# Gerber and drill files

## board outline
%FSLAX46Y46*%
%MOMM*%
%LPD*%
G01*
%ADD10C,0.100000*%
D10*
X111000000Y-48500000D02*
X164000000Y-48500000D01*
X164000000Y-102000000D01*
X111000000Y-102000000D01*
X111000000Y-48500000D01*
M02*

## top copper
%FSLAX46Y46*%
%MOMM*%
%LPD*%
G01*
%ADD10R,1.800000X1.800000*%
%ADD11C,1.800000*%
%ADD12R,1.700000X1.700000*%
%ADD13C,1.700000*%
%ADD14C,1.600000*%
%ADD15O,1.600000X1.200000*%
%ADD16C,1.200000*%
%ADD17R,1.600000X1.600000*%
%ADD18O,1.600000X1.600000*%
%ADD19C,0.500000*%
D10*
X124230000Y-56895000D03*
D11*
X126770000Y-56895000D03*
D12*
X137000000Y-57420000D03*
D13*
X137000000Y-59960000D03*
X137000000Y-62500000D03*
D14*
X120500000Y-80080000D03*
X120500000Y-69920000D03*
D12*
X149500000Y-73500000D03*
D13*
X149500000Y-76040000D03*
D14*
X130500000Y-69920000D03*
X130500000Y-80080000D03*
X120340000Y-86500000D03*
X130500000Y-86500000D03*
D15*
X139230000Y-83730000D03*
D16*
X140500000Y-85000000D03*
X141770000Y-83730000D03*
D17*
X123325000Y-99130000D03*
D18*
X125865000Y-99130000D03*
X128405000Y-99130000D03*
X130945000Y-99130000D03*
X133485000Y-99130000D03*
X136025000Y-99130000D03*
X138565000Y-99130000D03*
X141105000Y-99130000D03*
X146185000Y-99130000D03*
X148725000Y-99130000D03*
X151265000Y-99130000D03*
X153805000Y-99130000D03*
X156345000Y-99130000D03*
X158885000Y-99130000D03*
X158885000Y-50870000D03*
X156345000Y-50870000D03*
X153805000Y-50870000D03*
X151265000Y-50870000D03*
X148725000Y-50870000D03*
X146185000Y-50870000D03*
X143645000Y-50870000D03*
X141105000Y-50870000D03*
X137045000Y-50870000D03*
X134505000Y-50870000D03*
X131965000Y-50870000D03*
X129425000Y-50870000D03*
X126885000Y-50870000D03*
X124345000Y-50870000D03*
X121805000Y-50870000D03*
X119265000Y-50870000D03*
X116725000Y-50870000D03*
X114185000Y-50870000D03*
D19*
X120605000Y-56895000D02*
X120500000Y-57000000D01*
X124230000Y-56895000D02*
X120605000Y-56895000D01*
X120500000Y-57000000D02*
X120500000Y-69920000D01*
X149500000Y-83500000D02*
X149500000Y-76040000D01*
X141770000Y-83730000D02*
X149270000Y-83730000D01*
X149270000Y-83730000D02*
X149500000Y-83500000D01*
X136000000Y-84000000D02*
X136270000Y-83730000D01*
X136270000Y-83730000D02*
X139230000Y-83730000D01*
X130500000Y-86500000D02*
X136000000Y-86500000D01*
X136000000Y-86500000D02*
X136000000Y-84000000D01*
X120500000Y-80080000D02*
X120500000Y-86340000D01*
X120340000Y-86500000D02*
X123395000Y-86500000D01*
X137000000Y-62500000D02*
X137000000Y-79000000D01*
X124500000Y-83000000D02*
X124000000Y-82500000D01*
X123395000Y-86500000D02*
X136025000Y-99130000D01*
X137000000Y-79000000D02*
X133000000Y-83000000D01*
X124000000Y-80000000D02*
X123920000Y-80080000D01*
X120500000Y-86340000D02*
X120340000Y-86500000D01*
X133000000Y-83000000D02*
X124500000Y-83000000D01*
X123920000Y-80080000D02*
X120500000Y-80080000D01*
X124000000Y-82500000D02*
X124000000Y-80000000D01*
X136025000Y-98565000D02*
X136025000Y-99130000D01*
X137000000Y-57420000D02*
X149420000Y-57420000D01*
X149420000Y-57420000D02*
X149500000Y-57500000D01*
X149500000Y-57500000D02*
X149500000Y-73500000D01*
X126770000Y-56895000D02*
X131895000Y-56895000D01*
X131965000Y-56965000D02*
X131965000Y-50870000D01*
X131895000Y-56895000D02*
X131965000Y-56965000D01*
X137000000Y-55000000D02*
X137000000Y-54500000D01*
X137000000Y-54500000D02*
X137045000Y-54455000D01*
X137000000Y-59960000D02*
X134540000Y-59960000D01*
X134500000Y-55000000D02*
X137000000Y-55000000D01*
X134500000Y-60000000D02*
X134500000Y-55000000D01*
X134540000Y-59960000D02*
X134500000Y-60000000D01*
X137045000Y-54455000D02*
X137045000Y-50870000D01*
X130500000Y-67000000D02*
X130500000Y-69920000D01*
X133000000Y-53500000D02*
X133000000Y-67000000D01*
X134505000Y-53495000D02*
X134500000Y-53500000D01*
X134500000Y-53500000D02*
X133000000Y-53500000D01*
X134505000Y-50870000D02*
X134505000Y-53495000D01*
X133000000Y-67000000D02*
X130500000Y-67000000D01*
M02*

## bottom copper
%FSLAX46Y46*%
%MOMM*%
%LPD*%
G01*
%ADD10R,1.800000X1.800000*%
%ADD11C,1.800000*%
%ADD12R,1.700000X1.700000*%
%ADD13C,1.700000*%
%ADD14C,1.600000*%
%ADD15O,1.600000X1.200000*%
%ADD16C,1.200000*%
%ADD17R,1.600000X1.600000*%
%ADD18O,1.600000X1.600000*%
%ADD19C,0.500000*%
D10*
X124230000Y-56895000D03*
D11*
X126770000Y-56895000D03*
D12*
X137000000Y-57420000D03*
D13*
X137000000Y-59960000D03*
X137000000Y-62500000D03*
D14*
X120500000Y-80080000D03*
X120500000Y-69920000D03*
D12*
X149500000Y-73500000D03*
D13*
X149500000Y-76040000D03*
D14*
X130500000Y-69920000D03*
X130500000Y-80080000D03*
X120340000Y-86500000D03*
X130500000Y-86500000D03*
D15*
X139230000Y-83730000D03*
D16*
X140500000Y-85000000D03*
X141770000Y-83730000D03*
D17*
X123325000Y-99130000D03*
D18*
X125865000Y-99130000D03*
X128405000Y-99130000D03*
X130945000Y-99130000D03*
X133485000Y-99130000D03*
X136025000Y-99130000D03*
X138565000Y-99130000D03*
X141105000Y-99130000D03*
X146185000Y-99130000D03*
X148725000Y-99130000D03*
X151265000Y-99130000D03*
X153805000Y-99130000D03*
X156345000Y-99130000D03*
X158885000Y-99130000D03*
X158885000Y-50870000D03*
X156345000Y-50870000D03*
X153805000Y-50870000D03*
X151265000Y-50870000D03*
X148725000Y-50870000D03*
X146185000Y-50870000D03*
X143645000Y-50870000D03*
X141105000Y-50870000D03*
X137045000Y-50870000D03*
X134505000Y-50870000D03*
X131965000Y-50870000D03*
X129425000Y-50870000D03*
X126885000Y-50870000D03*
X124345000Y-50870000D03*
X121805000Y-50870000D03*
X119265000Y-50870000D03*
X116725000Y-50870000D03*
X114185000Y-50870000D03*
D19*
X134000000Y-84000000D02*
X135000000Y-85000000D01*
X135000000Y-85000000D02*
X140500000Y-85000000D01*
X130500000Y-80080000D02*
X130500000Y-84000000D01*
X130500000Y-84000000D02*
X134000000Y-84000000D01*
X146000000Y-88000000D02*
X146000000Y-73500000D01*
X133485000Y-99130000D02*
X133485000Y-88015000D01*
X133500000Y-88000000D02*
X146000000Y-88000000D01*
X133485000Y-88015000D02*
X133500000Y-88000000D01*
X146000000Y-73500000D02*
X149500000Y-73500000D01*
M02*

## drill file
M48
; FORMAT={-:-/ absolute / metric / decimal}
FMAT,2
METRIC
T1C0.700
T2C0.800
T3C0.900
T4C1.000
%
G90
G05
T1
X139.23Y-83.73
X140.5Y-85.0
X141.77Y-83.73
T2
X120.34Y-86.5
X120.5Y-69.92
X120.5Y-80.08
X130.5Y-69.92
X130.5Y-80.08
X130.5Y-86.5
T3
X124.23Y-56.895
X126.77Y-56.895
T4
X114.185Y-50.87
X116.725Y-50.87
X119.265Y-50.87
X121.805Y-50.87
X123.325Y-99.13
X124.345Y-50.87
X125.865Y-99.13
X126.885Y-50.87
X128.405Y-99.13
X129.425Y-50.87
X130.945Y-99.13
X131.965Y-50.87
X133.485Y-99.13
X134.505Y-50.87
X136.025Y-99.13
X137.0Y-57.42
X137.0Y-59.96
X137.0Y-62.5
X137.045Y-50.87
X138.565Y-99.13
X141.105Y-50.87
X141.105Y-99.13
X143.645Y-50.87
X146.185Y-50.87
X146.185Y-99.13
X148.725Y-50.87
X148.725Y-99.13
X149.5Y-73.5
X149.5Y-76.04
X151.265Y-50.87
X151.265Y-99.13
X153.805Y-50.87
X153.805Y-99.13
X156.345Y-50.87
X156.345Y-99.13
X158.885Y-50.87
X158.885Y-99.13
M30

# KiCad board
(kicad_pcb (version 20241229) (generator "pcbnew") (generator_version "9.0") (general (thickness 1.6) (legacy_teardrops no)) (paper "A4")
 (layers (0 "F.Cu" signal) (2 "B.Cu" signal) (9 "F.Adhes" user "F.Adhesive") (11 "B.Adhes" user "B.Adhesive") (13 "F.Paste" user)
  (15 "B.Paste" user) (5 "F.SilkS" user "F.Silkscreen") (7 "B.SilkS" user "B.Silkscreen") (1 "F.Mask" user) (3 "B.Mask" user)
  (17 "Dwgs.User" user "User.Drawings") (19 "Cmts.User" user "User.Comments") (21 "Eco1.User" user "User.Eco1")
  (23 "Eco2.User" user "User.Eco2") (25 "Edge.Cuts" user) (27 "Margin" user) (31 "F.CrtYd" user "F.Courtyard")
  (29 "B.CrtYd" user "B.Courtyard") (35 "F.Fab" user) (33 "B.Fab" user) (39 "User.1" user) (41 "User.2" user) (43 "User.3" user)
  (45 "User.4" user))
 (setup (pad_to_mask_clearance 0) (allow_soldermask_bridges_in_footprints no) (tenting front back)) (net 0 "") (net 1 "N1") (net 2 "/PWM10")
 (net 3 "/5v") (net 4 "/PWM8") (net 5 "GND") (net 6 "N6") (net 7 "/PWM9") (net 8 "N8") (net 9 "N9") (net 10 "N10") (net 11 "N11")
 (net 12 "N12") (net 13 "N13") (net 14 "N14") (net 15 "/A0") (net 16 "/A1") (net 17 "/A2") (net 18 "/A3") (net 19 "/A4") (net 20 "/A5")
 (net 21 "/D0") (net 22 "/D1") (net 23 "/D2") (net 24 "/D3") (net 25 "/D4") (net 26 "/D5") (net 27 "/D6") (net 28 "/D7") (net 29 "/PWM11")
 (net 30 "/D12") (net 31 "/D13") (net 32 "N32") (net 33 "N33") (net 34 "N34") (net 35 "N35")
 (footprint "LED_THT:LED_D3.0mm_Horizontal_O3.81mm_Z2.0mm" (layer "F.Cu") (at 124.23 56.895)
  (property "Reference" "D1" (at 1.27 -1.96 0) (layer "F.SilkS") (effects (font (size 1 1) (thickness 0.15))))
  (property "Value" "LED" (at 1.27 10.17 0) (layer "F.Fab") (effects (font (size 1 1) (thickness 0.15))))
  (pad "1" thru_hole rect (at 0 0) (size 1.8 1.8) (drill 0.9) (layers "*.Cu" "*.Mask") (remove_unused_layers no) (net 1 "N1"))
  (pad "2" thru_hole circle (at 2.54 0) (size 1.8 1.8) (drill 0.9) (layers "*.Cu" "*.Mask") (remove_unused_layers no) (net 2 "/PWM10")))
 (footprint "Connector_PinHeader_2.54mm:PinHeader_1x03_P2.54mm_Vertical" (layer "F.Cu") (at 137 57.42)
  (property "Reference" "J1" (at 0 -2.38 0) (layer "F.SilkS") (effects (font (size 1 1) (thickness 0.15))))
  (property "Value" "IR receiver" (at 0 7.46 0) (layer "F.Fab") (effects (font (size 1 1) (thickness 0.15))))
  (pad "1" thru_hole rect (at 0 0) (size 1.7 1.7) (drill 1) (layers "*.Cu" "*.Mask") (remove_unused_layers no) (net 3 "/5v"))
  (pad "2" thru_hole circle (at 0 2.54) (size 1.7 1.7) (drill 1) (layers "*.Cu" "*.Mask") (remove_unused_layers no) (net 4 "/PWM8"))
  (pad "3" thru_hole circle (at 0 5.08) (size 1.7 1.7) (drill 1) (layers "*.Cu" "*.Mask") (remove_unused_layers no) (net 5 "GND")))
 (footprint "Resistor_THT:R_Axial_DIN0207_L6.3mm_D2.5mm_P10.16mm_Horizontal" (layer "F.Cu") (at 120.5 80.08 90)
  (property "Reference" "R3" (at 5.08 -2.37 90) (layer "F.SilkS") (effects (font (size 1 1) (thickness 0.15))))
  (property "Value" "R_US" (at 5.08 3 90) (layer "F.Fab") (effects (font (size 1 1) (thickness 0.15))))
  (pad "1" thru_hole circle (at 0 0 90) (size 1.6 1.6) (drill 0.8) (layers "*.Cu" "*.Mask") (remove_unused_layers no) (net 5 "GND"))
  (pad "2" thru_hole circle (at 10.16 0 90) (size 1.6 1.6) (drill 0.8) (layers "*.Cu" "*.Mask") (remove_unused_layers no) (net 1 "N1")))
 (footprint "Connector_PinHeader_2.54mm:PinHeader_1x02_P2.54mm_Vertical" (layer "F.Cu") (at 149.5 73.5)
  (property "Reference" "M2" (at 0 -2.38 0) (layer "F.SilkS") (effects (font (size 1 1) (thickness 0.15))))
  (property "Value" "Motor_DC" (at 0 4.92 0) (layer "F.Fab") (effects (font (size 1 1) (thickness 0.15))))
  (pad "1" thru_hole rect (at 0 0) (size 1.7 1.7) (drill 1) (layers "*.Cu" "*.Mask") (remove_unused_layers no) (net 3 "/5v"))
  (pad "2" thru_hole circle (at 0 2.54) (size 1.7 1.7) (drill 1) (layers "*.Cu" "*.Mask") (remove_unused_layers no) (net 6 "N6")))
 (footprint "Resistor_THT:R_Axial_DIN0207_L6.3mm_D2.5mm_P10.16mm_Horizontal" (layer "F.Cu") (at 130.5 69.92 -90)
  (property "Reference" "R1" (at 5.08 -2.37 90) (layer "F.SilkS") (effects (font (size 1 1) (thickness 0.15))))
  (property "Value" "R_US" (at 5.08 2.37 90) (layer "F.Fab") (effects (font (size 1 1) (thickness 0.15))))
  (pad "1" thru_hole circle (at 0 0 270) (size 1.6 1.6) (drill 0.8) (layers "*.Cu" "*.Mask") (remove_unused_layers no) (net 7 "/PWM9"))
  (pad "2" thru_hole circle (at 10.16 0 270) (size 1.6 1.6) (drill 0.8) (layers "*.Cu" "*.Mask") (remove_unused_layers no) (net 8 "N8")))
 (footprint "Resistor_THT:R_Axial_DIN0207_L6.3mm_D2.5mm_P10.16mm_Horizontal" (layer "F.Cu") (at 120.34 86.5)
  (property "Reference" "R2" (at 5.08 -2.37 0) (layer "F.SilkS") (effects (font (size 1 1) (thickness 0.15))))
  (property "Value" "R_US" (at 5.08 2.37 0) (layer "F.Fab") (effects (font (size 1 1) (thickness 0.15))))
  (pad "1" thru_hole circle (at 0 0) (size 1.6 1.6) (drill 0.8) (layers "*.Cu" "*.Mask") (remove_unused_layers no) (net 5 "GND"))
  (pad "2" thru_hole circle (at 10.16 0) (size 1.6 1.6) (drill 0.8) (layers "*.Cu" "*.Mask") (remove_unused_layers no) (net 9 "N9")))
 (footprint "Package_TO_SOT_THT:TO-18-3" (layer "F.Cu") (at 139.23 83.73)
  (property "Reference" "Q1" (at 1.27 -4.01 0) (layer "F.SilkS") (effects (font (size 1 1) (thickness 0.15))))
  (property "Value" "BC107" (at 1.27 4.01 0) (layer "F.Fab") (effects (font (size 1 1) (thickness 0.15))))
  (pad "1" thru_hole oval (at 0 0) (size 1.6 1.2) (drill 0.7) (layers "*.Cu" "*.Mask") (remove_unused_layers no) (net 9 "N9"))
  (pad "2" thru_hole circle (at 1.27 1.27) (size 1.2 1.2) (drill 0.7) (layers "*.Cu" "*.Mask") (remove_unused_layers no) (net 8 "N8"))
  (pad "3" thru_hole circle (at 2.54 0) (size 1.2 1.2) (drill 0.7) (layers "*.Cu" "*.Mask") (remove_unused_layers no) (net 6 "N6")))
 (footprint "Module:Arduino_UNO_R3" (layer "B.Cu") (at 123.325 99.13)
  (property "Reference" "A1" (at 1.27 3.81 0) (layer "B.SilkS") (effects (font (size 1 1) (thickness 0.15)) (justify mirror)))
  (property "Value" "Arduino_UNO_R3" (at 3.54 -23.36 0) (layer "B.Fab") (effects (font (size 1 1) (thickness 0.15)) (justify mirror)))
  (pad "1" thru_hole rect (at 0 0 270) (size 1.6 1.6) (drill 1) (layers "*.Cu" "*.Mask") (remove_unused_layers no) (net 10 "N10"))
  (pad "2" thru_hole oval (at 2.54 0 270) (size 1.6 1.6) (drill 1) (layers "*.Cu" "*.Mask") (remove_unused_layers no) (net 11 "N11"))
  (pad "3" thru_hole oval (at 5.08 0 270) (size 1.6 1.6) (drill 1) (layers "*.Cu" "*.Mask") (remove_unused_layers no) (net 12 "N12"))
  (pad "4" thru_hole oval (at 7.62 0 270) (size 1.6 1.6) (drill 1) (layers "*.Cu" "*.Mask") (remove_unused_layers no) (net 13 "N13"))
  (pad "5" thru_hole oval (at 10.16 0 270) (size 1.6 1.6) (drill 1) (layers "*.Cu" "*.Mask") (remove_unused_layers no) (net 3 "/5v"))
  (pad "6" thru_hole oval (at 12.7 0 270) (size 1.6 1.6) (drill 1) (layers "*.Cu" "*.Mask") (remove_unused_layers no) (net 5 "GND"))
  (pad "7" thru_hole oval (at 15.24 0 270) (size 1.6 1.6) (drill 1) (layers "*.Cu" "*.Mask") (remove_unused_layers no) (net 5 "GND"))
  (pad "8" thru_hole oval (at 17.78 0 270) (size 1.6 1.6) (drill 1) (layers "*.Cu" "*.Mask") (remove_unused_layers no) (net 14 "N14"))
  (pad "9" thru_hole oval (at 22.86 0 270) (size 1.6 1.6) (drill 1) (layers "*.Cu" "*.Mask") (remove_unused_layers no) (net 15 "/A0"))
  (pad "10" thru_hole oval (at 25.4 0 270) (size 1.6 1.6) (drill 1) (layers "*.Cu" "*.Mask") (remove_unused_layers no) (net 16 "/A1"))
  (pad "11" thru_hole oval (at 27.94 0 270) (size 1.6 1.6) (drill 1) (layers "*.Cu" "*.Mask") (remove_unused_layers no) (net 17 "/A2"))
  (pad "12" thru_hole oval (at 30.48 0 270) (size 1.6 1.6) (drill 1) (layers "*.Cu" "*.Mask") (remove_unused_layers no) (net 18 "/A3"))
  (pad "13" thru_hole oval (at 33.02 0 270) (size 1.6 1.6) (drill 1) (layers "*.Cu" "*.Mask") (remove_unused_layers no) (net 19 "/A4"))
  (pad "14" thru_hole oval (at 35.56 0 270) (size 1.6 1.6) (drill 1) (layers "*.Cu" "*.Mask") (remove_unused_layers no) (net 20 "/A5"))
  (pad "15" thru_hole oval (at 35.56 -48.26 270) (size 1.6 1.6) (drill 1) (layers "*.Cu" "*.Mask") (remove_unused_layers no) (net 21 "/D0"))
  (pad "16" thru_hole oval (at 33.02 -48.26 270) (size 1.6 1.6) (drill 1) (layers "*.Cu" "*.Mask") (remove_unused_layers no) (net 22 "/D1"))
  (pad "17" thru_hole oval (at 30.48 -48.26 270) (size 1.6 1.6) (drill 1) (layers "*.Cu" "*.Mask") (remove_unused_layers no) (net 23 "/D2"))
  (pad "18" thru_hole oval (at 27.94 -48.26 270) (size 1.6 1.6) (drill 1) (layers "*.Cu" "*.Mask") (remove_unused_layers no) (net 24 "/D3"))
  (pad "19" thru_hole oval (at 25.4 -48.26 270) (size 1.6 1.6) (drill 1) (layers "*.Cu" "*.Mask") (remove_unused_layers no) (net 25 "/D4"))
  (pad "20" thru_hole oval (at 22.86 -48.26 270) (size 1.6 1.6) (drill 1) (layers "*.Cu" "*.Mask") (remove_unused_layers no) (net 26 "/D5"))
  (pad "21" thru_hole oval (at 20.32 -48.26 270) (size 1.6 1.6) (drill 1) (layers "*.Cu" "*.Mask") (remove_unused_layers no) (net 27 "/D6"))
  (pad "22" thru_hole oval (at 17.78 -48.26 270) (size 1.6 1.6) (drill 1) (layers "*.Cu" "*.Mask") (remove_unused_layers no) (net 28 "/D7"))
  (pad "23" thru_hole oval (at 13.72 -48.26 270) (size 1.6 1.6) (drill 1) (layers "*.Cu" "*.Mask") (remove_unused_layers no) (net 4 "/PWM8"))
  (pad "24" thru_hole oval (at 11.18 -48.26 270) (size 1.6 1.6) (drill 1) (layers "*.Cu" "*.Mask") (remove_unused_layers no) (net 7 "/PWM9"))
  (pad "25" thru_hole oval (at 8.64 -48.26 270) (size 1.6 1.6) (drill 1) (layers "*.Cu" "*.Mask") (remove_unused_layers no) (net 2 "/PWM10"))
  (pad "26" thru_hole oval (at 6.1 -48.26 270) (size 1.6 1.6) (drill 1) (layers "*.Cu" "*.Mask") (remove_unused_layers no) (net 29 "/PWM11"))
  (pad "27" thru_hole oval (at 3.56 -48.26 270) (size 1.6 1.6) (drill 1) (layers "*.Cu" "*.Mask") (remove_unused_layers no) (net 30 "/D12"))
  (pad "28" thru_hole oval (at 1.02 -48.26 270) (size 1.6 1.6) (drill 1) (layers "*.Cu" "*.Mask") (remove_unused_layers no) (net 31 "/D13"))
  (pad "29" thru_hole oval (at -1.52 -48.26 270) (size 1.6 1.6) (drill 1) (layers "*.Cu" "*.Mask") (remove_unused_layers no) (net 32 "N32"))
  (pad "30" thru_hole oval (at -4.06 -48.26 270) (size 1.6 1.6) (drill 1) (layers "*.Cu" "*.Mask") (remove_unused_layers no) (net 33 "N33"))
  (pad "31" thru_hole oval (at -6.6 -48.26 270) (size 1.6 1.6) (drill 1) (layers "*.Cu" "*.Mask") (remove_unused_layers no) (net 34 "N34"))
  (pad "32" thru_hole oval (at -9.14 -48.26 270) (size 1.6 1.6) (drill 1) (layers "*.Cu" "*.Mask") (remove_unused_layers no) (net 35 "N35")))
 (gr_rect (start 111 48.5) (end 164 102) (stroke (width 0.1) (type default)) (fill no) (layer "Edge.Cuts"))
 (segment (start 120.605 56.895) (end 120.5 57) (width 0.5) (layer "F.Cu") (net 1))
 (segment (start 124.23 56.895) (end 120.605 56.895) (width 0.5) (layer "F.Cu") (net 1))
 (segment (start 120.5 57) (end 120.5 69.92) (width 0.5) (layer "F.Cu") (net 1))
 (segment (start 149.5 83.5) (end 149.5 76.04) (width 0.5) (layer "F.Cu") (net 6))
 (segment (start 141.77 83.73) (end 149.27 83.73) (width 0.5) (layer "F.Cu") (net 6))
 (segment (start 149.27 83.73) (end 149.5 83.5) (width 0.5) (layer "F.Cu") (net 6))
 (segment (start 136 84) (end 136.27 83.73) (width 0.5) (layer "F.Cu") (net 9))
 (segment (start 136.27 83.73) (end 139.23 83.73) (width 0.5) (layer "F.Cu") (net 9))
 (segment (start 130.5 86.5) (end 136 86.5) (width 0.5) (layer "F.Cu") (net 9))
 (segment (start 136 86.5) (end 136 84) (width 0.5) (layer "F.Cu") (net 9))
 (segment (start 120.5 80.08) (end 120.5 86.34) (width 0.5) (layer "F.Cu") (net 5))
 (segment (start 120.34 86.5) (end 123.395 86.5) (width 0.5) (layer "F.Cu") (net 5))
 (segment (start 137 62.5) (end 137 79) (width 0.5) (layer "F.Cu") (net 5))
 (segment (start 124.5 83) (end 124 82.5) (width 0.5) (layer "F.Cu") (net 5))
 (segment (start 123.395 86.5) (end 136.025 99.13) (width 0.5) (layer "F.Cu") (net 5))
 (segment (start 137 79) (end 133 83) (width 0.5) (layer "F.Cu") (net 5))
 (segment (start 124 80) (end 123.92 80.08) (width 0.5) (layer "F.Cu") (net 5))
 (segment (start 120.5 86.34) (end 120.34 86.5) (width 0.5) (layer "F.Cu") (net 5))
 (segment (start 133 83) (end 124.5 83) (width 0.5) (layer "F.Cu") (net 5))
 (segment (start 123.92 80.08) (end 120.5 80.08) (width 0.5) (layer "F.Cu") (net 5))
 (segment (start 124 82.5) (end 124 80) (width 0.5) (layer "F.Cu") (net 5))
 (segment (start 136.025 98.565) (end 136.025 99.13) (width 0.5) (layer "F.Cu") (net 5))
 (segment (start 134 84) (end 135 85) (width 0.5) (layer "B.Cu") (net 8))
 (segment (start 135 85) (end 140.5 85) (width 0.5) (layer "B.Cu") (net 8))
 (segment (start 130.5 80.08) (end 130.5 84) (width 0.5) (layer "B.Cu") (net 8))
 (segment (start 130.5 84) (end 134 84) (width 0.5) (layer "B.Cu") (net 8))
 (segment (start 137 57.42) (end 149.42 57.42) (width 0.5) (layer "F.Cu") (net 3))
 (segment (start 149.42 57.42) (end 149.5 57.5) (width 0.5) (layer "F.Cu") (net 3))
 (segment (start 149.5 57.5) (end 149.5 73.5) (width 0.5) (layer "F.Cu") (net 3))
 (segment (start 146 88) (end 146 73.5) (width 0.5) (layer "B.Cu") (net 3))
 (segment (start 133.485 99.13) (end 133.485 88.015) (width 0.5) (layer "B.Cu") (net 3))
 (segment (start 133.5 88) (end 146 88) (width 0.5) (layer "B.Cu") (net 3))
 (segment (start 133.485 88.015) (end 133.5 88) (width 0.5) (layer "B.Cu") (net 3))
 (segment (start 146 73.5) (end 149.5 73.5) (width 0.5) (layer "B.Cu") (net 3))
 (segment (start 126.77 56.895) (end 131.895 56.895) (width 0.5) (layer "F.Cu") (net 2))
 (segment (start 131.965 56.965) (end 131.965 50.87) (width 0.5) (layer "F.Cu") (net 2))
 (segment (start 131.895 56.895) (end 131.965 56.965) (width 0.5) (layer "F.Cu") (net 2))
 (segment (start 137 55) (end 137 54.5) (width 0.5) (layer "F.Cu") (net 4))
 (segment (start 137 54.5) (end 137.045 54.455) (width 0.5) (layer "F.Cu") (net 4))
 (segment (start 137 59.96) (end 134.54 59.96) (width 0.5) (layer "F.Cu") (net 4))
 (segment (start 134.5 55) (end 137 55) (width 0.5) (layer "F.Cu") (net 4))
 (segment (start 134.5 60) (end 134.5 55) (width 0.5) (layer "F.Cu") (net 4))
 (segment (start 134.54 59.96) (end 134.5 60) (width 0.5) (layer "F.Cu") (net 4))
 (segment (start 137.045 54.455) (end 137.045 50.87) (width 0.5) (layer "F.Cu") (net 4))
 (segment (start 130.5 67) (end 130.5 69.92) (width 0.5) (layer "F.Cu") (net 7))
 (segment (start 133 53.5) (end 133 67) (width 0.5) (layer "F.Cu") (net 7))
 (segment (start 134.505 53.495) (end 134.5 53.5) (width 0.5) (layer "F.Cu") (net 7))
 (segment (start 134.5 53.5) (end 133 53.5) (width 0.5) (layer "F.Cu") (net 7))
 (segment (start 134.505 50.87) (end 134.505 53.495) (width 0.5) (layer "F.Cu") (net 7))
 (segment (start 133 67) (end 130.5 67) (width 0.5) (layer "F.Cu") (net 7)))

